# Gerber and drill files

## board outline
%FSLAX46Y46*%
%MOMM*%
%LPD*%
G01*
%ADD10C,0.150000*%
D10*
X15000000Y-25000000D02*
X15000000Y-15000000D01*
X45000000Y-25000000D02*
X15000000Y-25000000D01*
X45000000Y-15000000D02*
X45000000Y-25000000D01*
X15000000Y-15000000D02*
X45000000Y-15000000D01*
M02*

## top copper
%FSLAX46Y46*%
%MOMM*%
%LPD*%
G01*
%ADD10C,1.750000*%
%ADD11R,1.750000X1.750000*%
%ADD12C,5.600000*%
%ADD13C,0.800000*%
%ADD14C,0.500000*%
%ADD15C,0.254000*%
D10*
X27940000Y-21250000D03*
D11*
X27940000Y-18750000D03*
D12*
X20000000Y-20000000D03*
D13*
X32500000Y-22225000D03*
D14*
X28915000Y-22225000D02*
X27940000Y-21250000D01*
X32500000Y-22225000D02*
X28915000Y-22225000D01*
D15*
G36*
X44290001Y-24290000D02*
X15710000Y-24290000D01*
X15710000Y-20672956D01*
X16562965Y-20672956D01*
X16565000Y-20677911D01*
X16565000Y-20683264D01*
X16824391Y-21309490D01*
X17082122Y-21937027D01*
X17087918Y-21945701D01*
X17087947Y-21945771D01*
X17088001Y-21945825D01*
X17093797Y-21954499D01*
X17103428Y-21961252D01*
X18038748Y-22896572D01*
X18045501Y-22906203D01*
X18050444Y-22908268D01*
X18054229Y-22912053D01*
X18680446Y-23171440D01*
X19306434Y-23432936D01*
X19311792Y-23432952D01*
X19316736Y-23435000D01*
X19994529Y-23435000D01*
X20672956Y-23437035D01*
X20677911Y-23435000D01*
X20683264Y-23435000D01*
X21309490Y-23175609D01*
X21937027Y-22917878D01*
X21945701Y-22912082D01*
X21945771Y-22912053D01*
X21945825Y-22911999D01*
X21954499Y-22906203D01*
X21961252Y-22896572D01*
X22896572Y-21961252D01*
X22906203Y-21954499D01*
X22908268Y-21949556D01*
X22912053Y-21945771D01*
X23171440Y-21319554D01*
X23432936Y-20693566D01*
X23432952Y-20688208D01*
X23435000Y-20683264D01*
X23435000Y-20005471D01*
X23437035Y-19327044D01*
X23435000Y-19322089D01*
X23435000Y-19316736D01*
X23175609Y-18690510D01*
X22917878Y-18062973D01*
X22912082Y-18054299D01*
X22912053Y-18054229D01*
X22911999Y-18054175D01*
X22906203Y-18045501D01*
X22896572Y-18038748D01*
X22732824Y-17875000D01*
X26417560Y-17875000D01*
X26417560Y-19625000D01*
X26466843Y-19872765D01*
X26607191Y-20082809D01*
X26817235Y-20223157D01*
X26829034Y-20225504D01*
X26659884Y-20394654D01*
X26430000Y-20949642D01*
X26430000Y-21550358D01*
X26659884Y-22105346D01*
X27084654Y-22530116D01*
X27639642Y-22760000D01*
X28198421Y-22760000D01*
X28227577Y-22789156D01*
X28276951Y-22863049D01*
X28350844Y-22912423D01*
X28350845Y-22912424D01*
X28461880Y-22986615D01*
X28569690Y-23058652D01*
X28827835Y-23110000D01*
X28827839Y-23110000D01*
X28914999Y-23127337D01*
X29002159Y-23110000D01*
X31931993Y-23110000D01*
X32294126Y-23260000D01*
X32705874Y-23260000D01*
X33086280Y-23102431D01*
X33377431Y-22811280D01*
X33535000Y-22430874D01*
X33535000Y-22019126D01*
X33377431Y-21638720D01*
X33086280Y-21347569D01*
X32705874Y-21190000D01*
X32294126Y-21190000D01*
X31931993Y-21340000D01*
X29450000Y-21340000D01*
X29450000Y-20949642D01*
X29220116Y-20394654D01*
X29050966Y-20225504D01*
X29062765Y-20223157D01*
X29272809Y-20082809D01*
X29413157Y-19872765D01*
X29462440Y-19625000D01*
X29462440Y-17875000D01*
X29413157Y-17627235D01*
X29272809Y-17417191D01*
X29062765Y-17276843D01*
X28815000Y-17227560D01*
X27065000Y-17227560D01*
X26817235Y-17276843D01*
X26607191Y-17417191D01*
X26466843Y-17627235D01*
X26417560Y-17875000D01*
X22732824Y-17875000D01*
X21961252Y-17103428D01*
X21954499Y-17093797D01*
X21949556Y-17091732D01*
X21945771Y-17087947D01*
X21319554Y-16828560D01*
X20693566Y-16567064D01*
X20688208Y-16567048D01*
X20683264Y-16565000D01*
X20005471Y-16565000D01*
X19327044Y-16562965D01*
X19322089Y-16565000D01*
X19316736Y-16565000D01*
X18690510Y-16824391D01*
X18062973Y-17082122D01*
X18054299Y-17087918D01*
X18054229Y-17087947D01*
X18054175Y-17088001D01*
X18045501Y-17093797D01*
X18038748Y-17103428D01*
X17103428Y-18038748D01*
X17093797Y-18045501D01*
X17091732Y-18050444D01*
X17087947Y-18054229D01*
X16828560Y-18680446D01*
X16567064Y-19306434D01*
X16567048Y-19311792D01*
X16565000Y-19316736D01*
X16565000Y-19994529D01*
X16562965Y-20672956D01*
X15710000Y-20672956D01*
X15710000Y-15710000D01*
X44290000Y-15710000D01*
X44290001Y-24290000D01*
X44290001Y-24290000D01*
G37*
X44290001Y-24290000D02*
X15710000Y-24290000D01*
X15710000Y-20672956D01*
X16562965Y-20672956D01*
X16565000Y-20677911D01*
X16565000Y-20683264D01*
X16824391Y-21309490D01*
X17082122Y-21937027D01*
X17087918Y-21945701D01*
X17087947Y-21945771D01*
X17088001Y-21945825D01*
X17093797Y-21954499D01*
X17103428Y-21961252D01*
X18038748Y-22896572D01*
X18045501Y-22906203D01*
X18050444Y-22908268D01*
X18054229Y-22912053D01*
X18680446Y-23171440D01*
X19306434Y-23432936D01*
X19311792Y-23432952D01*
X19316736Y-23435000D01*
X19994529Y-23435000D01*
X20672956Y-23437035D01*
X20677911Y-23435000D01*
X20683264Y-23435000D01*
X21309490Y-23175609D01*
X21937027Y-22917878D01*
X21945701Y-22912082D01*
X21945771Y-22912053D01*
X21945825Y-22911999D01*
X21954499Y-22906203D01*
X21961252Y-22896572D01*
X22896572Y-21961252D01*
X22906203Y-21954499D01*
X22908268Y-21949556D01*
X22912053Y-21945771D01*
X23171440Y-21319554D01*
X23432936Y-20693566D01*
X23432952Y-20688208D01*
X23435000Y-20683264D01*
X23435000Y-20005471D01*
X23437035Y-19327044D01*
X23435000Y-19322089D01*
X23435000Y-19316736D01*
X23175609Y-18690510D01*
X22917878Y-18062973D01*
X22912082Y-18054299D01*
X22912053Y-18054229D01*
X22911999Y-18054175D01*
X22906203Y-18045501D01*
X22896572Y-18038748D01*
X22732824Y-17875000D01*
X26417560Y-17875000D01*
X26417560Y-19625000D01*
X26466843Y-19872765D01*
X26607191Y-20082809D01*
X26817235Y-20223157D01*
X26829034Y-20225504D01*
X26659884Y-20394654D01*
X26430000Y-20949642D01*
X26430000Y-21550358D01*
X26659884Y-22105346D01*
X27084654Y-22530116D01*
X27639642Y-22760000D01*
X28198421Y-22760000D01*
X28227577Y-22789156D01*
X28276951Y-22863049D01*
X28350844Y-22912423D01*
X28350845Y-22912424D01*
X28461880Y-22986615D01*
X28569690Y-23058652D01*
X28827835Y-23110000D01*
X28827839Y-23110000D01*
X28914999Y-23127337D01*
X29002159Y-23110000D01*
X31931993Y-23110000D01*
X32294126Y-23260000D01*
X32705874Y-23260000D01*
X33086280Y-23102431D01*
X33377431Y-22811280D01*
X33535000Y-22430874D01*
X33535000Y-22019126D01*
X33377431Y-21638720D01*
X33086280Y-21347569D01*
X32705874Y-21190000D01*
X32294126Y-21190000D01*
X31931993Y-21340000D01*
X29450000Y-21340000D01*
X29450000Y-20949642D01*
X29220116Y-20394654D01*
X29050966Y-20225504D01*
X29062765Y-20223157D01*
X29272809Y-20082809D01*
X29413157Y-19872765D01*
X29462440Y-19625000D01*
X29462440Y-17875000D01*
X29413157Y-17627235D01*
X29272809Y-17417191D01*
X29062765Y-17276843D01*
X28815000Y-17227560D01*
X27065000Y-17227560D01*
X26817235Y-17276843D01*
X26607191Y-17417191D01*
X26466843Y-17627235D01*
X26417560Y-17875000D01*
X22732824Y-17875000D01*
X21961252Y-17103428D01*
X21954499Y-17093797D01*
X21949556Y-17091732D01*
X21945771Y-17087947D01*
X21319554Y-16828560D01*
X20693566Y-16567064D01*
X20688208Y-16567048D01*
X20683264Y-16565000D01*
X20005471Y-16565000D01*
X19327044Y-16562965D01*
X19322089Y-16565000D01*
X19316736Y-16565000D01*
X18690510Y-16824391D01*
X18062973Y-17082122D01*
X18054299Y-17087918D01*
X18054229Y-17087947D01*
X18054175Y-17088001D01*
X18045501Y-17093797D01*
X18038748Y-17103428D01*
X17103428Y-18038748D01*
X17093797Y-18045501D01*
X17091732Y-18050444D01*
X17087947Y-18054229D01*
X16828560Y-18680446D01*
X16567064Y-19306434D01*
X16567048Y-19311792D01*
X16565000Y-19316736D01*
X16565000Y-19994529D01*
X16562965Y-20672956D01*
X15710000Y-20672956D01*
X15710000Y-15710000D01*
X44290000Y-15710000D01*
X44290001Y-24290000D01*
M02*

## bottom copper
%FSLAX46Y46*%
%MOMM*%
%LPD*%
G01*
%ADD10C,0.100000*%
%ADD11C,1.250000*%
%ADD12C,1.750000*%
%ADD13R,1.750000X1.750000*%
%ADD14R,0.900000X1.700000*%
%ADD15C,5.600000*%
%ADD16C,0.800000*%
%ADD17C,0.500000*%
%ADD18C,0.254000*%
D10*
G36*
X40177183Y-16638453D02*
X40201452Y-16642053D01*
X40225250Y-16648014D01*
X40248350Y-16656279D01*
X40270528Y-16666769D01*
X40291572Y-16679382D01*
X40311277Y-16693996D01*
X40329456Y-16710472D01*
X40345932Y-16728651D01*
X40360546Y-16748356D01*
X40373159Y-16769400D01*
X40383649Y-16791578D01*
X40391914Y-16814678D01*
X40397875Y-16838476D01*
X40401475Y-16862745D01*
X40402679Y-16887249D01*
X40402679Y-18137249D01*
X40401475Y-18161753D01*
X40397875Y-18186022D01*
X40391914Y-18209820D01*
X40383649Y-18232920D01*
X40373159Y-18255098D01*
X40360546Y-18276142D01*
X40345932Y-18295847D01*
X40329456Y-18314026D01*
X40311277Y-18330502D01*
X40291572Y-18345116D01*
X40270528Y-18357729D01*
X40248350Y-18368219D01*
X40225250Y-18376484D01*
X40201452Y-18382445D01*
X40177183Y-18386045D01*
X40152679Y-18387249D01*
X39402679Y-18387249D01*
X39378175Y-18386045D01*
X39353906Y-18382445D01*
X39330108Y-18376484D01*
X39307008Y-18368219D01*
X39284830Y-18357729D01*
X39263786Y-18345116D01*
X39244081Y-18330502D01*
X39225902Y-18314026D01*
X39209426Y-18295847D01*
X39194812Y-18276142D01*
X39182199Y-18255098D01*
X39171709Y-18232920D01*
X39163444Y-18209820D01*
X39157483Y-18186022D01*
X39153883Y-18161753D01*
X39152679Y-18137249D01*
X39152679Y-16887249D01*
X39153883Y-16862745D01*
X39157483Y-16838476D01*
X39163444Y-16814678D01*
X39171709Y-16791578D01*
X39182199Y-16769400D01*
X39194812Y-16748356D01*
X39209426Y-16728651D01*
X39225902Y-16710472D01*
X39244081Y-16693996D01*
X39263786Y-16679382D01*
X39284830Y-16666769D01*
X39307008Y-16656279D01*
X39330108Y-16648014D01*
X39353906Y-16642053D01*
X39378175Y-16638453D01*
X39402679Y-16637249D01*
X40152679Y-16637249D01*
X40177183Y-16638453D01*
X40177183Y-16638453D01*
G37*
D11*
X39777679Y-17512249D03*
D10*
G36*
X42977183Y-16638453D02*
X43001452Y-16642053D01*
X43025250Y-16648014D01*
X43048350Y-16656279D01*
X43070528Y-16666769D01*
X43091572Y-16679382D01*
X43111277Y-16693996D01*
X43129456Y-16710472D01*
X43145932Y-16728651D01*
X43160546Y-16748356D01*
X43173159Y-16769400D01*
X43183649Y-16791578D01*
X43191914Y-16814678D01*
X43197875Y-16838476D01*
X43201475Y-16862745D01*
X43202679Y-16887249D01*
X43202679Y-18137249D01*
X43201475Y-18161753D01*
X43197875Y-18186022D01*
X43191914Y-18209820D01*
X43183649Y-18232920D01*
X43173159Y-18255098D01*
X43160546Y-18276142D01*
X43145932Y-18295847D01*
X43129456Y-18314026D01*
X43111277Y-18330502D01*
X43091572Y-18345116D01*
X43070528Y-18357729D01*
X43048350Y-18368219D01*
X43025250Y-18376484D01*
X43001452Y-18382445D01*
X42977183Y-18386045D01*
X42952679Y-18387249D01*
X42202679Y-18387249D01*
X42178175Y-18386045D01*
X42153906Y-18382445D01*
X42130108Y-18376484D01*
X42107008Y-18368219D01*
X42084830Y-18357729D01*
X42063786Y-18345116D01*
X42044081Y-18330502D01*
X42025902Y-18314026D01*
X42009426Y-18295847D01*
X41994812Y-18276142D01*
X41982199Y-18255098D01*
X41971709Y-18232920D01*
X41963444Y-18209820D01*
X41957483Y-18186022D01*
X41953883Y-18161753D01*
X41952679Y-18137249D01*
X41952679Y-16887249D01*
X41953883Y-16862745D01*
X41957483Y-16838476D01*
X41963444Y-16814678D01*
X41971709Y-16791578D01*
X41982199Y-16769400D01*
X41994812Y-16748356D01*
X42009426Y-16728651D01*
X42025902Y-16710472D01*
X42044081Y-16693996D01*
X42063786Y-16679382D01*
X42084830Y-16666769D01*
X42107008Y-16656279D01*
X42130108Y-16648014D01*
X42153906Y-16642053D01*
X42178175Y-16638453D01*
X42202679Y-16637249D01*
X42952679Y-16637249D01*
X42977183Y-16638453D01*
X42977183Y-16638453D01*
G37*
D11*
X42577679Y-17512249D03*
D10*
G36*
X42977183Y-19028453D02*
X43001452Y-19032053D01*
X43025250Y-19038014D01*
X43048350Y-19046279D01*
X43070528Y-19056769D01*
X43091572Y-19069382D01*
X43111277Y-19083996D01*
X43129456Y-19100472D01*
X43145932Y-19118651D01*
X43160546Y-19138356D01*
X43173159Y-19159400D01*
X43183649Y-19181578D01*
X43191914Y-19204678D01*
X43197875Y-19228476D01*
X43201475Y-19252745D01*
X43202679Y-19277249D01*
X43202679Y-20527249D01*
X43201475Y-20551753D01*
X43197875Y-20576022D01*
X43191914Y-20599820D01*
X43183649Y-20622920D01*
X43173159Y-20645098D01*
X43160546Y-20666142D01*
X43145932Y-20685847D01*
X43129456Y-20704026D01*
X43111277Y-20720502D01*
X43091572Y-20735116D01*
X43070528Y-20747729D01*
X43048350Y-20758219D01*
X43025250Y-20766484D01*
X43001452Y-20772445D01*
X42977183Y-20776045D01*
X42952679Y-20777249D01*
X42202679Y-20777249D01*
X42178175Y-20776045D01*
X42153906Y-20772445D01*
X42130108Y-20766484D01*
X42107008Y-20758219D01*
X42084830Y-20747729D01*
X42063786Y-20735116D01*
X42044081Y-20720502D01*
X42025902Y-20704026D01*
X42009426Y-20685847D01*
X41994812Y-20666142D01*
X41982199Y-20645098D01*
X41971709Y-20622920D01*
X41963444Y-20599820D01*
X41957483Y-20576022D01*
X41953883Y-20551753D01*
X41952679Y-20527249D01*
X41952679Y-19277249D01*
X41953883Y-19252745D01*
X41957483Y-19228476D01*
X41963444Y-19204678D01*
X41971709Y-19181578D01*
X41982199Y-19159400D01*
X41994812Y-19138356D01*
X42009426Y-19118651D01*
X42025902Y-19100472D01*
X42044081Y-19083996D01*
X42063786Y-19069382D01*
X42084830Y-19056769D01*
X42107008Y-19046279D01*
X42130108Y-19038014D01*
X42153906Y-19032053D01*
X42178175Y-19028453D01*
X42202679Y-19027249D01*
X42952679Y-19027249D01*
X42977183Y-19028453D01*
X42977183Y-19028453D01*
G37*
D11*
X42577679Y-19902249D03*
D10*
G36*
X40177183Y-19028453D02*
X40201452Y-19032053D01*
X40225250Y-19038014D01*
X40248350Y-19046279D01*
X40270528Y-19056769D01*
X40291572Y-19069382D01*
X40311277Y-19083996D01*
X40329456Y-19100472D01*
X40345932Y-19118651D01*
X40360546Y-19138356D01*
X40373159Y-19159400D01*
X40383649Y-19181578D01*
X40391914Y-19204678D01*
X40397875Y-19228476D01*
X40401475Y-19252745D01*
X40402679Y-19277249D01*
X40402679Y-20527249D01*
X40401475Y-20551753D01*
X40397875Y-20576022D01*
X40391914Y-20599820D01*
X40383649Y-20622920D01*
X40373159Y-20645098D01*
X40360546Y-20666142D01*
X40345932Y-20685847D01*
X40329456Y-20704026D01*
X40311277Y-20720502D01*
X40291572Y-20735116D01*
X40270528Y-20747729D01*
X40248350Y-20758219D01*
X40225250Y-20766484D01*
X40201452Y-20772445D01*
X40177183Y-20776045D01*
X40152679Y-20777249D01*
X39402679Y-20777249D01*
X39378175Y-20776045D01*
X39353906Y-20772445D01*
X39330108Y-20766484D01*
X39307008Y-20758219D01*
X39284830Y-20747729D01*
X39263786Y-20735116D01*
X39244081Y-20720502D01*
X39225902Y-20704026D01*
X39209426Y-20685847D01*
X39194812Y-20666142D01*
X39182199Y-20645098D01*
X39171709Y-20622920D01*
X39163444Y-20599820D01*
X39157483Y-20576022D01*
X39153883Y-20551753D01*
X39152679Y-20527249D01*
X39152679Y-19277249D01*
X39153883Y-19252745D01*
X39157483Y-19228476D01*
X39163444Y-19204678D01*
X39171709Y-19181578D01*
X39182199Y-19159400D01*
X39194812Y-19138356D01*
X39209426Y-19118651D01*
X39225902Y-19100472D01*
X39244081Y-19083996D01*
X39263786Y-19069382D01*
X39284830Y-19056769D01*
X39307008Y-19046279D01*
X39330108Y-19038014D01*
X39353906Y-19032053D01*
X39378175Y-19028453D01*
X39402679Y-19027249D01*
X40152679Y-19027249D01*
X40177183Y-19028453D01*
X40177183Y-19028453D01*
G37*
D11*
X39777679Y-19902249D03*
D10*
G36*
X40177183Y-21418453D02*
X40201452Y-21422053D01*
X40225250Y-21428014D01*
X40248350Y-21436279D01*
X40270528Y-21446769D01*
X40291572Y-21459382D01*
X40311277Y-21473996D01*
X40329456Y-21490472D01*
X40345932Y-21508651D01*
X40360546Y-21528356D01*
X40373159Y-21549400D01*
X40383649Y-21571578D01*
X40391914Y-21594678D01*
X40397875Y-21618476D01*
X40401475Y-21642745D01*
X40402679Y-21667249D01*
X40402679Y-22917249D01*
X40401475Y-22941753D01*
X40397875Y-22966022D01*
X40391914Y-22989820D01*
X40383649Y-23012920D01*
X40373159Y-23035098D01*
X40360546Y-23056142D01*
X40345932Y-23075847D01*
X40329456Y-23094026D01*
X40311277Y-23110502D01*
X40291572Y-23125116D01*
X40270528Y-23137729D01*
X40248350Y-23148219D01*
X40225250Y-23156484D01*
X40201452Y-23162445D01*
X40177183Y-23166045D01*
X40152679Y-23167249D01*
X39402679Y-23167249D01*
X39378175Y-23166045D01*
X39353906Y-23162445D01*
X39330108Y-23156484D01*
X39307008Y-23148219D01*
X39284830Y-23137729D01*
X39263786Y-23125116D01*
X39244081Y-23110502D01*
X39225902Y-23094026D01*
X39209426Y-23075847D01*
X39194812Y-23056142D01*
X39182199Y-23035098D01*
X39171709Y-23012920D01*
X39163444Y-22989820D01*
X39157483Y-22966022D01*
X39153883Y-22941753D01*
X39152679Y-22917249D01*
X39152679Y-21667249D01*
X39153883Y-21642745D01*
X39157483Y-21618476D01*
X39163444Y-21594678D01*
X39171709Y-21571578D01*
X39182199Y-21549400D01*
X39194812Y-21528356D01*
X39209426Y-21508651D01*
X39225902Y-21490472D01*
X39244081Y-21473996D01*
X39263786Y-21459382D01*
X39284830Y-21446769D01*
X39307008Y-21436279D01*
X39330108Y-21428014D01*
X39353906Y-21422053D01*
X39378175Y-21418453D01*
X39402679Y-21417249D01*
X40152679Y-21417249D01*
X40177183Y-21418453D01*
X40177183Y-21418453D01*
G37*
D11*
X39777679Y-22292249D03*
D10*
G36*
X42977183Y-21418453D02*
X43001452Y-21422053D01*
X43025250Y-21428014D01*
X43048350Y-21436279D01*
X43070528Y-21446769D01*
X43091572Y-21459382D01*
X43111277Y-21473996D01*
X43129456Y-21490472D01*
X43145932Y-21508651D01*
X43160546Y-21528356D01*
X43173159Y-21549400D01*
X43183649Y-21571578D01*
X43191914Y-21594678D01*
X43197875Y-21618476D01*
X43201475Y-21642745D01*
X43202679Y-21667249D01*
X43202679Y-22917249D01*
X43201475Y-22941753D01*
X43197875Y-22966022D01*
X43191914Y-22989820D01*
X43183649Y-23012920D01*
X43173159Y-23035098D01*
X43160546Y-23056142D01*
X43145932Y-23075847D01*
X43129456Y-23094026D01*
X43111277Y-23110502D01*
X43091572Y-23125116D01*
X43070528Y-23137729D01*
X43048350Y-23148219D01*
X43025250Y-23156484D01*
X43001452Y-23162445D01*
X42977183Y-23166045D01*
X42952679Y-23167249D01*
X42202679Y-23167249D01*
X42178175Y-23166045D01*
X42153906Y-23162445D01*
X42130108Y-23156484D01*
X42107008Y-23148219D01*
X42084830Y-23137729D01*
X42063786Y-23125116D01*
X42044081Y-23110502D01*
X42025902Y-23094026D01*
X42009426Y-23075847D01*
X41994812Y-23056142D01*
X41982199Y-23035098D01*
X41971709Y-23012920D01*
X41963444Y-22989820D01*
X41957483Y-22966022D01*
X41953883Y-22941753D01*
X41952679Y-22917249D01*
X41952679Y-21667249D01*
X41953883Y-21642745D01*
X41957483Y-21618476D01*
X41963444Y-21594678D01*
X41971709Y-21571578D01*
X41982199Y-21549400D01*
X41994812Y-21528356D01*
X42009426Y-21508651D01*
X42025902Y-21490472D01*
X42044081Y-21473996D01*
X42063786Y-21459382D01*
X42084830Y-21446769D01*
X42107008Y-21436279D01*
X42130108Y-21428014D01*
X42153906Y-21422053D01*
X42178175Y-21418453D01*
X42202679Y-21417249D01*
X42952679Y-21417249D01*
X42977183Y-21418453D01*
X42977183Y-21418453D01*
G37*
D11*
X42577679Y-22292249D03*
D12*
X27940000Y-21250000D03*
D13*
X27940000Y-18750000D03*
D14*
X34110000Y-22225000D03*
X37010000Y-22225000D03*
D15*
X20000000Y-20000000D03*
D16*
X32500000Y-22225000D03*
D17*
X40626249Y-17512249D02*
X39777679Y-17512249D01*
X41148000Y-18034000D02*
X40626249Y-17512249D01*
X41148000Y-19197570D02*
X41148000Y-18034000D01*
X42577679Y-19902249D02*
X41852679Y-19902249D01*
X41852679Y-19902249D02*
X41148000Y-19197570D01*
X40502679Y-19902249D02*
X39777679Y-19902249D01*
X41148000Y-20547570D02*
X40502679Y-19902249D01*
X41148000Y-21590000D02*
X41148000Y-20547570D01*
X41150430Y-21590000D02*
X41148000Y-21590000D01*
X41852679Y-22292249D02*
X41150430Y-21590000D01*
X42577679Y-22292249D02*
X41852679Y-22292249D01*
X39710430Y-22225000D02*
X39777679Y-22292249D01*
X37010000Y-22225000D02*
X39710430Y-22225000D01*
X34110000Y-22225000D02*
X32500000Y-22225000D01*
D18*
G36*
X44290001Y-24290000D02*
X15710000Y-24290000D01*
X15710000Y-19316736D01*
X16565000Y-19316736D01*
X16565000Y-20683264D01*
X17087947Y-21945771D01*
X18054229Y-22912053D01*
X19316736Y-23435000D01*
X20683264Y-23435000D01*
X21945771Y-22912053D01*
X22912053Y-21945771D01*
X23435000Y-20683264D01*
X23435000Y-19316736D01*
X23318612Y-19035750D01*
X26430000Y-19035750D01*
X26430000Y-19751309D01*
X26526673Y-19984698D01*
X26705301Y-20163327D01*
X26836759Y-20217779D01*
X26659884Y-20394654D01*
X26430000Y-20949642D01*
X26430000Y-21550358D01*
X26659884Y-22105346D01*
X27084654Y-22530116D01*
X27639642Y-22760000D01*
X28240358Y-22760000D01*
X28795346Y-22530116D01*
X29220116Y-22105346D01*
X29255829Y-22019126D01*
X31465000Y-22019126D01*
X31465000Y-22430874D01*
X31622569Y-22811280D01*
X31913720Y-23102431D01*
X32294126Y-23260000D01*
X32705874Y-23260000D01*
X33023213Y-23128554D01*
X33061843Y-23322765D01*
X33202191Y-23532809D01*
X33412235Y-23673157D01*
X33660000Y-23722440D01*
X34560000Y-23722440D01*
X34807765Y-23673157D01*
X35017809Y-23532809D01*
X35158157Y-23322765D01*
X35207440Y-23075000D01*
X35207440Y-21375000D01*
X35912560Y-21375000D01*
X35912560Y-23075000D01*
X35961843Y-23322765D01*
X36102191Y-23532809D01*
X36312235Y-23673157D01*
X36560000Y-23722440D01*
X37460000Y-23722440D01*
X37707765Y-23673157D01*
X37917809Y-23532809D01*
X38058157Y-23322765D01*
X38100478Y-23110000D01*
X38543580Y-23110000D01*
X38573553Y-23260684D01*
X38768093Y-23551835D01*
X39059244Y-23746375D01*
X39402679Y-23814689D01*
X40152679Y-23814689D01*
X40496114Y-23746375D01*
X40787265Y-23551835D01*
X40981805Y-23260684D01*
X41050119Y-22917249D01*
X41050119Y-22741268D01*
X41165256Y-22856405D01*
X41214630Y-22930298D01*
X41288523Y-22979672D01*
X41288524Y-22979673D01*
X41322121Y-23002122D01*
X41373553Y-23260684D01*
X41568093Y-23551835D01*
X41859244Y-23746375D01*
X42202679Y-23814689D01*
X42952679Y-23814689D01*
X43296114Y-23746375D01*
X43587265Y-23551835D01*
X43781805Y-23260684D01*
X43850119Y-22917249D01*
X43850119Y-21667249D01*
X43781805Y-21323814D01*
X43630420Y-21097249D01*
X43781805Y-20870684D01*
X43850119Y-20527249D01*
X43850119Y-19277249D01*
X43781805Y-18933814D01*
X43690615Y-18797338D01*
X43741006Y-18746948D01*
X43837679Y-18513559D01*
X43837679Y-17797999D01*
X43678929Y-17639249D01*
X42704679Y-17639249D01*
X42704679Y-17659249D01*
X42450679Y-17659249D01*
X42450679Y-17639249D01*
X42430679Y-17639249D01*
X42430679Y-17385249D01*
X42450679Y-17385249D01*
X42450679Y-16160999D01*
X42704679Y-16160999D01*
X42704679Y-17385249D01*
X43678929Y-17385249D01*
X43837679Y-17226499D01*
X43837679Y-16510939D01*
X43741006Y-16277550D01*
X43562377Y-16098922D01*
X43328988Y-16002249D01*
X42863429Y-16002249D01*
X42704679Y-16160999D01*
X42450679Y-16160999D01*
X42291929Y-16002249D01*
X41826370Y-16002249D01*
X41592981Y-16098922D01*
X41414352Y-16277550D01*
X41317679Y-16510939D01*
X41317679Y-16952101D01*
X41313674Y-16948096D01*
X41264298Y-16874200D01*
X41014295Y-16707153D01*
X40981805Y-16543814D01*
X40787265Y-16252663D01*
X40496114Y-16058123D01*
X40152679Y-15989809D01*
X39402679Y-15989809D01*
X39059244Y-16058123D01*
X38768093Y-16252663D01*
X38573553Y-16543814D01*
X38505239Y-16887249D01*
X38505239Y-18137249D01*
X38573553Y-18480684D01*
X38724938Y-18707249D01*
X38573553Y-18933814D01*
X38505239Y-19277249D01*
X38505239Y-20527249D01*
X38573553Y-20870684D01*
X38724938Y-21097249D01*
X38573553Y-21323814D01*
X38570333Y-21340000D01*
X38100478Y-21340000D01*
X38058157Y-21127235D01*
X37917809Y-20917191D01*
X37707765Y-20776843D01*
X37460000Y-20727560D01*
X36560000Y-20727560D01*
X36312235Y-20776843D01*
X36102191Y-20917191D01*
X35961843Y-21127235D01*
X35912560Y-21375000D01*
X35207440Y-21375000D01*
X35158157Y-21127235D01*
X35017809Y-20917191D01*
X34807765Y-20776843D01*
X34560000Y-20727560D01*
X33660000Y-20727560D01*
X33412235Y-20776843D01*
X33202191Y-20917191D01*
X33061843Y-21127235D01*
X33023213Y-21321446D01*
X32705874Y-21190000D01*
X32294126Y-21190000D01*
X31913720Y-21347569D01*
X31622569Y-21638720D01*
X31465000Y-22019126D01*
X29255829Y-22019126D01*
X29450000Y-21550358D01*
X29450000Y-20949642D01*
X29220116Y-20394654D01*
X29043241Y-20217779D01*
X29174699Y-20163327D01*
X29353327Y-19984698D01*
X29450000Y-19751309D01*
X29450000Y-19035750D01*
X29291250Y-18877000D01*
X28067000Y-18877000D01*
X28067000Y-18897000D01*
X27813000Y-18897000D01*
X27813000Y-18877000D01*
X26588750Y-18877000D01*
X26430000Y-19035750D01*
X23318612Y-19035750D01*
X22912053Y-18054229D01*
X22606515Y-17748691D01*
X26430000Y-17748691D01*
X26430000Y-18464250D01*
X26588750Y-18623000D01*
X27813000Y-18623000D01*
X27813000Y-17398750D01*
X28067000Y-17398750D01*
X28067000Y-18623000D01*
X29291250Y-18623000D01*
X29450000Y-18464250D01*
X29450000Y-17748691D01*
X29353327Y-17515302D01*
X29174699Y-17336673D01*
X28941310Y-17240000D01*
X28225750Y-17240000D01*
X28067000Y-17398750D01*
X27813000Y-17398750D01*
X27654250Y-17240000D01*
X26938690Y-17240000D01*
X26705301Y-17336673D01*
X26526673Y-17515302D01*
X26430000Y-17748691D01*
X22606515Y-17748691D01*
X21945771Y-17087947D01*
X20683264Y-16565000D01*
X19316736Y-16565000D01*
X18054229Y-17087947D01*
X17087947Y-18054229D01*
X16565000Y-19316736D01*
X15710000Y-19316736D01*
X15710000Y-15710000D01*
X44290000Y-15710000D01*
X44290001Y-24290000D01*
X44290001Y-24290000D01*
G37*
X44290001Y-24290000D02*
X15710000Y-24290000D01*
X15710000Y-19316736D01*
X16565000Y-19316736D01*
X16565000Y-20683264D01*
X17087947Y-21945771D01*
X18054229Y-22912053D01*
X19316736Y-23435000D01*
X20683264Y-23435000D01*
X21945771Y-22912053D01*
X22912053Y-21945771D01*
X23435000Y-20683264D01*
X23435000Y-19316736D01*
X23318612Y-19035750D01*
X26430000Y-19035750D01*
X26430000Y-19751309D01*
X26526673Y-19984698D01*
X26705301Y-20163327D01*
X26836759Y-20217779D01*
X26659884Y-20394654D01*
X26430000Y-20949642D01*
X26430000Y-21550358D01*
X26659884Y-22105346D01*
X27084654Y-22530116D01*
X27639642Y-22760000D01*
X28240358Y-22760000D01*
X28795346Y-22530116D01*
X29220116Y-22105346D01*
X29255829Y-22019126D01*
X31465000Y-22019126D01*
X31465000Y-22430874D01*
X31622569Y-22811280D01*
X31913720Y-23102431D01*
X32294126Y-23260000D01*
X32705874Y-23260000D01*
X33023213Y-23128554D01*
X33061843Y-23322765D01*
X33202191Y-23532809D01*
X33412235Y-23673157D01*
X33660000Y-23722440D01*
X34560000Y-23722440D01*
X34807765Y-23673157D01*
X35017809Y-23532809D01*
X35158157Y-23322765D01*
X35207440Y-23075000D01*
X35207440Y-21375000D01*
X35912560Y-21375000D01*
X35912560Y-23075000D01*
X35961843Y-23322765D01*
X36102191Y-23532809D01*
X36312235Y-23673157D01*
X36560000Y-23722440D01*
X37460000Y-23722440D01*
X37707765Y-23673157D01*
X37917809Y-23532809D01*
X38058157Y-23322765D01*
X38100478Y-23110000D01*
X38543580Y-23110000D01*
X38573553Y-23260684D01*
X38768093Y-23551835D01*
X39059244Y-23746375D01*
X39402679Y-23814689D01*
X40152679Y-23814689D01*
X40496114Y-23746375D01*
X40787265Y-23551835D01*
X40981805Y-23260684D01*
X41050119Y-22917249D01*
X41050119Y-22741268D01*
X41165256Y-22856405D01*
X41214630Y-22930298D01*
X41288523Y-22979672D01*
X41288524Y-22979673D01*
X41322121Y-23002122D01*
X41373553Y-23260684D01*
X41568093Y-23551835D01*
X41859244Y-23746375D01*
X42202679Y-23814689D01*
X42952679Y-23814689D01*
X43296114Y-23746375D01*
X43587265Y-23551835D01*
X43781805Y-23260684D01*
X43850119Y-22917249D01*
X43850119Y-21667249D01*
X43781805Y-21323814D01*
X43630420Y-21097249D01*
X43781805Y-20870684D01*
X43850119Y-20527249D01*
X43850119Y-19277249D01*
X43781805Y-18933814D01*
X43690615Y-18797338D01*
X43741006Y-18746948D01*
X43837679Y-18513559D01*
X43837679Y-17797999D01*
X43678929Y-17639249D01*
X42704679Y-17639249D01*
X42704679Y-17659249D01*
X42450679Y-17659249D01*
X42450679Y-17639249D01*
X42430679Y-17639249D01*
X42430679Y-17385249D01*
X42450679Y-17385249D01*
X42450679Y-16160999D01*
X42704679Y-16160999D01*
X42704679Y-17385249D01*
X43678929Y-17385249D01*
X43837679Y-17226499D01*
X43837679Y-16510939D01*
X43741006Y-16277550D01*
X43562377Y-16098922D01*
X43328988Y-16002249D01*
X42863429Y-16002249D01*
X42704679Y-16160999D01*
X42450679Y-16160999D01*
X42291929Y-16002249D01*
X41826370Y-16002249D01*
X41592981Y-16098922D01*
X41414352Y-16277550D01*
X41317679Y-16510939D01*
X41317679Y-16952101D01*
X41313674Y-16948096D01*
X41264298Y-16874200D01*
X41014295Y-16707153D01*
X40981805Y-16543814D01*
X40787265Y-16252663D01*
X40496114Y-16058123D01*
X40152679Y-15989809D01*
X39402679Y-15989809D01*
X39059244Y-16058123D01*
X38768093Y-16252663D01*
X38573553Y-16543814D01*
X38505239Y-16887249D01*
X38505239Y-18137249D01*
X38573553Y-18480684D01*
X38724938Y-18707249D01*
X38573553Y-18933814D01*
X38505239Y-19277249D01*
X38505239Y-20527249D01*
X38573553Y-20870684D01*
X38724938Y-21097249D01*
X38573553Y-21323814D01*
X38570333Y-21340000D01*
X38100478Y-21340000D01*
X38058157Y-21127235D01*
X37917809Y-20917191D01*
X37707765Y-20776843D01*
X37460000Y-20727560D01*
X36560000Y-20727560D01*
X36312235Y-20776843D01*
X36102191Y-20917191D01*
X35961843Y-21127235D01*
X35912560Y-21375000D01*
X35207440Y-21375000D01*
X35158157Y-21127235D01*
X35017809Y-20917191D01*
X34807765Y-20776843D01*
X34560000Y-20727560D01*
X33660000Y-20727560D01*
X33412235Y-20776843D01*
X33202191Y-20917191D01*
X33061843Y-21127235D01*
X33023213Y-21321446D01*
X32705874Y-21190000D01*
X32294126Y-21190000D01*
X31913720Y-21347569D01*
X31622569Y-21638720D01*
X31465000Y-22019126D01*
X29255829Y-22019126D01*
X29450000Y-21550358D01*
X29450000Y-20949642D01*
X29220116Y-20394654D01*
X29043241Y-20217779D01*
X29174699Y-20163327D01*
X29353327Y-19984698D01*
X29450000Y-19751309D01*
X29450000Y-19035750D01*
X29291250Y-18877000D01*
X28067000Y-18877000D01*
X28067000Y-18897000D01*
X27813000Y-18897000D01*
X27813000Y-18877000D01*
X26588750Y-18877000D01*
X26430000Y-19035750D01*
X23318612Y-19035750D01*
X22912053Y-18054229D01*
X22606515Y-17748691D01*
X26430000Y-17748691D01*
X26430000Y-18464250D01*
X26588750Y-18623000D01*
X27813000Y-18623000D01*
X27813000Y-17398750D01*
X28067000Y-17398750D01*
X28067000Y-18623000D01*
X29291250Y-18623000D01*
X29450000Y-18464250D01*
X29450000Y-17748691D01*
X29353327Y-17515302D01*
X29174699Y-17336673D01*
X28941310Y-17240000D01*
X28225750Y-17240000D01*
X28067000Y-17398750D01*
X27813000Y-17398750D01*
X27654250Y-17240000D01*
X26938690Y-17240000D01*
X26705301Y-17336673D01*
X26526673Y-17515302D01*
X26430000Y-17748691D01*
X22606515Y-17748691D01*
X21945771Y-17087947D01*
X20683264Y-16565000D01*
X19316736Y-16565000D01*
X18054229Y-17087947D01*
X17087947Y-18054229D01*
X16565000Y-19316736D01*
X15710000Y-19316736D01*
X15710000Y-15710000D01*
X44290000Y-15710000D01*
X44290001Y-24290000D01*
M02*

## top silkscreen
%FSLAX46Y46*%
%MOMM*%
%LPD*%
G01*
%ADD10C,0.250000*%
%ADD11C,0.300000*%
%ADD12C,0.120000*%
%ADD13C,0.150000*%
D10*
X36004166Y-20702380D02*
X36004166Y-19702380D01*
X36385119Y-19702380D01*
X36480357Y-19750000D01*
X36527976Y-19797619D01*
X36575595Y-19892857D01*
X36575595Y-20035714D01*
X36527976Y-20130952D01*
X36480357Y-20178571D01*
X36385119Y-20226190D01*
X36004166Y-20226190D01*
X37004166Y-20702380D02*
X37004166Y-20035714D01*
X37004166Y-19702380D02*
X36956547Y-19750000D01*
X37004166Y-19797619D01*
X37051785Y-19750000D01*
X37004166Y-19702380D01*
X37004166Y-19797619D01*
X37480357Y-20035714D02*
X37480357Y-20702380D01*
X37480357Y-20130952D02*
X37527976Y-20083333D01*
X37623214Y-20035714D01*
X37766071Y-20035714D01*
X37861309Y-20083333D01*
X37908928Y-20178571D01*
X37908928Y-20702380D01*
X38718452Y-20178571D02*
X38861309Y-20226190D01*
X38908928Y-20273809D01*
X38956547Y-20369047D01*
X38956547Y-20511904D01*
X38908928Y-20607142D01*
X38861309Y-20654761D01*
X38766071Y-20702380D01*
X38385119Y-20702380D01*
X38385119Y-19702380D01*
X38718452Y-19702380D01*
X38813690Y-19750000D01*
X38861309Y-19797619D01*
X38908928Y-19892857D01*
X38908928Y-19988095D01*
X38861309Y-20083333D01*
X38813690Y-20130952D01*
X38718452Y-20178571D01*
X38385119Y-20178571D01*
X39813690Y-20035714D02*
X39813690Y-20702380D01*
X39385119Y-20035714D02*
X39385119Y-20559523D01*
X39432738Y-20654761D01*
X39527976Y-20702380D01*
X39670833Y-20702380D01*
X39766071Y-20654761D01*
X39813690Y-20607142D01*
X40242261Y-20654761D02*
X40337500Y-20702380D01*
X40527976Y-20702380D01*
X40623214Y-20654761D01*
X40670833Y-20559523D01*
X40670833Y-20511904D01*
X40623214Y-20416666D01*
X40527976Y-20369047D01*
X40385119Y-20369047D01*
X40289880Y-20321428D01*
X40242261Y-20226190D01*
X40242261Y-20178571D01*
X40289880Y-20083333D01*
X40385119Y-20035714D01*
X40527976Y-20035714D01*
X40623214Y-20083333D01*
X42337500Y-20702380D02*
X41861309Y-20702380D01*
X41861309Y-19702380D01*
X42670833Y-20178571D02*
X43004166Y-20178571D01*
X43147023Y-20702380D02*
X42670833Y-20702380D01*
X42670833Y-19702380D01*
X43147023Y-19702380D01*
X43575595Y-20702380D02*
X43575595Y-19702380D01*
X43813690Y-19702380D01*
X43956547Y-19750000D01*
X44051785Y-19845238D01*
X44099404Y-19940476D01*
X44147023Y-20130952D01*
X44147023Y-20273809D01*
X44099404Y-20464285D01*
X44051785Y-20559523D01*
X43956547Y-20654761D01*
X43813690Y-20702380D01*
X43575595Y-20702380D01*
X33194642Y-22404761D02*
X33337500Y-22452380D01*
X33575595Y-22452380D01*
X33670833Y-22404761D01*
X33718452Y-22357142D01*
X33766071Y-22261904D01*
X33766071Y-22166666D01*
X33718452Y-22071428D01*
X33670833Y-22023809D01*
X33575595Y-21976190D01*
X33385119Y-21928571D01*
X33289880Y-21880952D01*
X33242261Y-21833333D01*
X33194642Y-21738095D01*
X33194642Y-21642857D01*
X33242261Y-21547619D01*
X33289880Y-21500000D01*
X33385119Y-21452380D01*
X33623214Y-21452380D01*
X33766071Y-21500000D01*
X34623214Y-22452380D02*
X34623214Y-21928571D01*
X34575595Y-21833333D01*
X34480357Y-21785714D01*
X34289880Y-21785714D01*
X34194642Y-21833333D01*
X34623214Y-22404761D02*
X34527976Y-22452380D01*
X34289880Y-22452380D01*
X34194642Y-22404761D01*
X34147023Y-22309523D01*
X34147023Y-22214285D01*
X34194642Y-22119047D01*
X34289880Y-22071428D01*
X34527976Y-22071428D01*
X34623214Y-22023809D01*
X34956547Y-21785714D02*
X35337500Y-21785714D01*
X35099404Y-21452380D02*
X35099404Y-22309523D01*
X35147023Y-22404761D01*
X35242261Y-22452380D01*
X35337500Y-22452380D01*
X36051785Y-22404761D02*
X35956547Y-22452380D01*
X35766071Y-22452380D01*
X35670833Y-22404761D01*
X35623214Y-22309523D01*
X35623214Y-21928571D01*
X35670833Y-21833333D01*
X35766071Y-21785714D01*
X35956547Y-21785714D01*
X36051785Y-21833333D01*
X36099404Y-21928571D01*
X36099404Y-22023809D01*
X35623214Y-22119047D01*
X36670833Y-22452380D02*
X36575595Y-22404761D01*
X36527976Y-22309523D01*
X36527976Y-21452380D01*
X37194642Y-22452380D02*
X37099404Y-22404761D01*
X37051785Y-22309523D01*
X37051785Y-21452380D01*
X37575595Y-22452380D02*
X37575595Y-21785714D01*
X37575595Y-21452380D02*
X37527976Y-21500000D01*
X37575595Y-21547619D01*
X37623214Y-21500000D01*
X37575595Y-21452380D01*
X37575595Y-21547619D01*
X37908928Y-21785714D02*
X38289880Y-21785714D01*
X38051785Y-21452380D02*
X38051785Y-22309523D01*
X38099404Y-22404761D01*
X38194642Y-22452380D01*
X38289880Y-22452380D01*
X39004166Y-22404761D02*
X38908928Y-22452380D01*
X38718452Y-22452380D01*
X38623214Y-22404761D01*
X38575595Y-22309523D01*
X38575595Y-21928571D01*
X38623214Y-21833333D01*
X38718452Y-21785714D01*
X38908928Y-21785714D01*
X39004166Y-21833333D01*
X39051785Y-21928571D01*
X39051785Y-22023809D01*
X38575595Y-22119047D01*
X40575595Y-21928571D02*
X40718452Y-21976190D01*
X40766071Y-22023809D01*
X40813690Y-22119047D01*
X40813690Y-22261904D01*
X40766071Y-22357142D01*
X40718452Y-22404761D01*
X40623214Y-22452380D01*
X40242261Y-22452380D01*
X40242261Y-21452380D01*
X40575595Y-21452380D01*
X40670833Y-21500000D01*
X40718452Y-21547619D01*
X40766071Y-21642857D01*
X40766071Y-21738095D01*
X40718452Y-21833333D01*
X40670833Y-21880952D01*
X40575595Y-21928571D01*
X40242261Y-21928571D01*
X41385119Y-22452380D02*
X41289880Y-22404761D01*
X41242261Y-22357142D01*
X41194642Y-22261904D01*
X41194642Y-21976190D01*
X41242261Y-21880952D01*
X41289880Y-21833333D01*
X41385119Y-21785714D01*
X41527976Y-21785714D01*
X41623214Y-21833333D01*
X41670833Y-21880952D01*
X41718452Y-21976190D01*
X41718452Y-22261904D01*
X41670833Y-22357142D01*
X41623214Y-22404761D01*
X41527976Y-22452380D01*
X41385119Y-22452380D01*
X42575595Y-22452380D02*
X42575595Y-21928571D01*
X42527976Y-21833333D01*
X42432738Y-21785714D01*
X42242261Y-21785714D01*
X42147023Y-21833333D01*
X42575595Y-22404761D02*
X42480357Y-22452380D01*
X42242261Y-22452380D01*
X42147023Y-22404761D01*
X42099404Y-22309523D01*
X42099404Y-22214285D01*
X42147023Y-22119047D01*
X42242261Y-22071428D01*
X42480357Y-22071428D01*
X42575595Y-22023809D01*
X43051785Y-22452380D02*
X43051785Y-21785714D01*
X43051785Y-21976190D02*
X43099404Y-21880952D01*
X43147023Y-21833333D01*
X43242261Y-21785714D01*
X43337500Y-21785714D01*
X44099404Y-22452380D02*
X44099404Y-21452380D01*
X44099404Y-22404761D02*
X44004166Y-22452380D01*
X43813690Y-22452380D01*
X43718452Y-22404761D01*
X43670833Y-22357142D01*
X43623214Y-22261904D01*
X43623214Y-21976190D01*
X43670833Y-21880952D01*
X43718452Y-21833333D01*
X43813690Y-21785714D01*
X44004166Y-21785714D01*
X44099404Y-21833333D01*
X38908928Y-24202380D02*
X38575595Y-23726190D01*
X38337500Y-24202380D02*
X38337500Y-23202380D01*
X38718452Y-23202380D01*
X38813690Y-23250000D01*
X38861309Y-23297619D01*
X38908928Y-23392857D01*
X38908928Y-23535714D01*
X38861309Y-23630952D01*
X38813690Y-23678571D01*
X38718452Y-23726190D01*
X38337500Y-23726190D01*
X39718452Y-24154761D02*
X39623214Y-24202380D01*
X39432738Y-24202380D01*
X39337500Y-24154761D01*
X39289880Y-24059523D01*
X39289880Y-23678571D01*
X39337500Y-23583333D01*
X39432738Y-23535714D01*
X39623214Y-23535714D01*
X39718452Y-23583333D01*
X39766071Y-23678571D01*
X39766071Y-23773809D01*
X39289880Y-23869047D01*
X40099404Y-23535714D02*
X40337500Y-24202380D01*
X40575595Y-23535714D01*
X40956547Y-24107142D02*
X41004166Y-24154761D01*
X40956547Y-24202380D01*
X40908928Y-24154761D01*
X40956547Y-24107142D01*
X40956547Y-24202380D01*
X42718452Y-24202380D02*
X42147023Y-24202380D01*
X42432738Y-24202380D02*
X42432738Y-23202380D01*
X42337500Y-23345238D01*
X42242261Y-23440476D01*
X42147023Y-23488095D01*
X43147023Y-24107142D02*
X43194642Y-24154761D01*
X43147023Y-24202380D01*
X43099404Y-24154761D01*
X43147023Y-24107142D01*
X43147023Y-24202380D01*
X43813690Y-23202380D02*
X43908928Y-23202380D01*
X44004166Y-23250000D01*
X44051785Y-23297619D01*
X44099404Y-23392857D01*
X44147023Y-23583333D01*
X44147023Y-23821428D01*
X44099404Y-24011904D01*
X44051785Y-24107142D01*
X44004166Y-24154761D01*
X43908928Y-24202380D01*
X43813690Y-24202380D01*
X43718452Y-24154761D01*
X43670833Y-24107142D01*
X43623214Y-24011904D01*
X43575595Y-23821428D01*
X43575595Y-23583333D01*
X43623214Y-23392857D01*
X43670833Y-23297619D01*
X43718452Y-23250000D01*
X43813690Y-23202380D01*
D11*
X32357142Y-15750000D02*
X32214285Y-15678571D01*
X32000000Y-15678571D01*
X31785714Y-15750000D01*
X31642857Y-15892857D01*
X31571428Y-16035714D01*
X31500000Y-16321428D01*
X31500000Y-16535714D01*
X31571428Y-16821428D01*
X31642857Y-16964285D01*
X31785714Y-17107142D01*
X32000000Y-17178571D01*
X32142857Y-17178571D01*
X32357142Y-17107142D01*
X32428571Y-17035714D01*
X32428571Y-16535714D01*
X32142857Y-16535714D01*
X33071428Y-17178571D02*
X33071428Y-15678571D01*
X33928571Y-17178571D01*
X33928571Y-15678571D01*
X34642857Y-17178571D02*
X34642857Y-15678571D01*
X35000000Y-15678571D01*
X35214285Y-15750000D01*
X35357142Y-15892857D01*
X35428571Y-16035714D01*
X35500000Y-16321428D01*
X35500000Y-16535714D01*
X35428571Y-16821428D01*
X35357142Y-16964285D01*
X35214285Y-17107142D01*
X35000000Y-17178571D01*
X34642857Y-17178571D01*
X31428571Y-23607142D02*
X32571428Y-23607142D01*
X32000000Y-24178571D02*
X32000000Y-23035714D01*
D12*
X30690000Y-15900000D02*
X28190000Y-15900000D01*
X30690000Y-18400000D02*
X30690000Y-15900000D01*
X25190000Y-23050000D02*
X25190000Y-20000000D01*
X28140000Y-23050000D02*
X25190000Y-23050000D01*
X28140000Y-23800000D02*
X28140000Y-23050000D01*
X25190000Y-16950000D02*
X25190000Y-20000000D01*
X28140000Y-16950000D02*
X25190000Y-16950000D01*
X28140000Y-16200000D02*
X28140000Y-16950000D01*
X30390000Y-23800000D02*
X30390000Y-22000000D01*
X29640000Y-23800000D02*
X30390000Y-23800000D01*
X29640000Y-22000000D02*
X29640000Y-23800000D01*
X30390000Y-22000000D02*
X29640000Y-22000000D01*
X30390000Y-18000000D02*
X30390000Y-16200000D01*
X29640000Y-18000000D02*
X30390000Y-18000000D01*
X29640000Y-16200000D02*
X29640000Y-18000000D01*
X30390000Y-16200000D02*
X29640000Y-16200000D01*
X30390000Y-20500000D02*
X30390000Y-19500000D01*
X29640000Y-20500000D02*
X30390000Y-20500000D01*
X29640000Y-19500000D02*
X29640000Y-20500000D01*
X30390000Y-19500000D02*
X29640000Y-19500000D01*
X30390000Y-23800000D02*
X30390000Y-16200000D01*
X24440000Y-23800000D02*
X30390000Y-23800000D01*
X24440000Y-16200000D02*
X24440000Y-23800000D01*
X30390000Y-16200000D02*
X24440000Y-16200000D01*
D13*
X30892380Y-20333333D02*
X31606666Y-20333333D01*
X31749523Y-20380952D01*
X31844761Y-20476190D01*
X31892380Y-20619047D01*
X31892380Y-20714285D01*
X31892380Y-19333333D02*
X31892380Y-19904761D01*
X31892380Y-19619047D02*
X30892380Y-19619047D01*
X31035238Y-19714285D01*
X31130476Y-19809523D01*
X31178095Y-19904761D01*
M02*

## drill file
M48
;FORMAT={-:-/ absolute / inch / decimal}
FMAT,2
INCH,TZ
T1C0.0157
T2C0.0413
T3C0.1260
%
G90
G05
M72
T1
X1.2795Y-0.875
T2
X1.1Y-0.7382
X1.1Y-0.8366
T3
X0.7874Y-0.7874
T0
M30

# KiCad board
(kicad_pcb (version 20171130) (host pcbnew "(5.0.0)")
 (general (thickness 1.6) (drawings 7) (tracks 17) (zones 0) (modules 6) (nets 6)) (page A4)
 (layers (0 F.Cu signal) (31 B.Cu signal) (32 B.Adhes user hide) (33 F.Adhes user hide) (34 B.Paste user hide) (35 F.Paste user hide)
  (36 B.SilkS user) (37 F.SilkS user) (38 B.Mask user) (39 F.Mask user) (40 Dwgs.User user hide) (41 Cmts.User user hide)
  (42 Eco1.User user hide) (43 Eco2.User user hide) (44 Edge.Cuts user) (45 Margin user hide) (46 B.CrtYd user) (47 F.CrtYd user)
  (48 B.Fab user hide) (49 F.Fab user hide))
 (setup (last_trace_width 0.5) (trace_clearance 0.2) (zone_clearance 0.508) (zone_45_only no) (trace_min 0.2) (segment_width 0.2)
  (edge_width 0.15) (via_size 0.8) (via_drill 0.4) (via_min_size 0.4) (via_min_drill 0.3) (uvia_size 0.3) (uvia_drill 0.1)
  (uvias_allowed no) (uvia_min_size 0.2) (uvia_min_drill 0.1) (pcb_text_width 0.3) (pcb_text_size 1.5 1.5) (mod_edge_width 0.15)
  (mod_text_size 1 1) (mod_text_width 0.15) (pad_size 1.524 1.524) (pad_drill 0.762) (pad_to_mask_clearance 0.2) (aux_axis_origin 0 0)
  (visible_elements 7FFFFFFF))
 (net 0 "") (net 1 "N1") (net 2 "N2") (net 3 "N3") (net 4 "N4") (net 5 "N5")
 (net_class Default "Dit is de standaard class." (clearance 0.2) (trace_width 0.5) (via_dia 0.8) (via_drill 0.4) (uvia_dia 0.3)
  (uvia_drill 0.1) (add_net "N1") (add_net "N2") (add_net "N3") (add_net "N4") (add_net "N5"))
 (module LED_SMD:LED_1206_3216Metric (layer B.Cu) (at 41.177679 17.512249)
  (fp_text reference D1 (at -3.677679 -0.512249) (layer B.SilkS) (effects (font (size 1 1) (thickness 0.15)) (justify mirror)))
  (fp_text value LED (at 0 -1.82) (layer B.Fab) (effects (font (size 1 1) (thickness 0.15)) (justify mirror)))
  (pad 1 smd roundrect (at -1.4 0) (size 1.25 1.75) (layers B.Cu B.Paste B.Mask) (roundrect_rratio 0.2) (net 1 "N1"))
  (pad 2 smd roundrect (at 1.4 0) (size 1.25 1.75) (layers B.Cu B.Paste B.Mask) (roundrect_rratio 0.2) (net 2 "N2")))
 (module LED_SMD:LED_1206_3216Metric (layer B.Cu) (at 41.177679 19.902249)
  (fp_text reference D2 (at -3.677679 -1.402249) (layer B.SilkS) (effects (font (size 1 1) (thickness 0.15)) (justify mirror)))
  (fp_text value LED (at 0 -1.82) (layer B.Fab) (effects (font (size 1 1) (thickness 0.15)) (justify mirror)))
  (pad 2 smd roundrect (at 1.4 0) (size 1.25 1.75) (layers B.Cu B.Paste B.Mask) (roundrect_rratio 0.2) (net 1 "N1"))
  (pad 1 smd roundrect (at -1.4 0) (size 1.25 1.75) (layers B.Cu B.Paste B.Mask) (roundrect_rratio 0.2) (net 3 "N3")))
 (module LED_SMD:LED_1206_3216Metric (layer B.Cu) (at 41.177679 22.292249)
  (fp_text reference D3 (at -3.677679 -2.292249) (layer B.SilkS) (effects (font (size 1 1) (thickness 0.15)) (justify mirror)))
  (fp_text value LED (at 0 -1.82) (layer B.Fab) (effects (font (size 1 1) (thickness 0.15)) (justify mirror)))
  (pad 1 smd roundrect (at -1.4 0) (size 1.25 1.75) (layers B.Cu B.Paste B.Mask) (roundrect_rratio 0.2) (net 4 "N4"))
  (pad 2 smd roundrect (at 1.4 0) (size 1.25 1.75) (layers B.Cu B.Paste B.Mask) (roundrect_rratio 0.2) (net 3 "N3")))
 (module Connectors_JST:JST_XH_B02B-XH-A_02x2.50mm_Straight (layer F.Cu) (at 27.94 18.75 270)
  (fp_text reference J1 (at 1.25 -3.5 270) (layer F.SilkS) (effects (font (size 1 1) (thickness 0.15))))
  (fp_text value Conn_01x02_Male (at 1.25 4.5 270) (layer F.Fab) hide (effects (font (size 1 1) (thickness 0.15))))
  (fp_line (start -2.85 -2.75) (end -2.85 -0.25) (layer F.SilkS) (width 0.12))
  (fp_line (start -0.35 -2.75) (end -2.85 -2.75) (layer F.SilkS) (width 0.12))
  (fp_line (start 4.3 2.75) (end 1.25 2.75) (layer F.SilkS) (width 0.12))
  (fp_line (start 4.3 -0.2) (end 4.3 2.75) (layer F.SilkS) (width 0.12))
  (fp_line (start 5.05 -0.2) (end 4.3 -0.2) (layer F.SilkS) (width 0.12))
  (fp_line (start -1.8 2.75) (end 1.25 2.75) (layer F.SilkS) (width 0.12))
  (fp_line (start -1.8 -0.2) (end -1.8 2.75) (layer F.SilkS) (width 0.12))
  (fp_line (start -2.55 -0.2) (end -1.8 -0.2) (layer F.SilkS) (width 0.12))
  (fp_line (start 5.05 -2.45) (end 3.25 -2.45) (layer F.SilkS) (width 0.12))
  (fp_line (start 5.05 -1.7) (end 5.05 -2.45) (layer F.SilkS) (width 0.12))
  (fp_line (start 3.25 -1.7) (end 5.05 -1.7) (layer F.SilkS) (width 0.12))
  (fp_line (start 3.25 -2.45) (end 3.25 -1.7) (layer F.SilkS) (width 0.12))
  (fp_line (start -0.75 -2.45) (end -2.55 -2.45) (layer F.SilkS) (width 0.12))
  (fp_line (start -0.75 -1.7) (end -0.75 -2.45) (layer F.SilkS) (width 0.12))
  (fp_line (start -2.55 -1.7) (end -0.75 -1.7) (layer F.SilkS) (width 0.12))
  (fp_line (start -2.55 -2.45) (end -2.55 -1.7) (layer F.SilkS) (width 0.12))
  (fp_line (start 1.75 -2.45) (end 0.75 -2.45) (layer F.SilkS) (width 0.12))
  (fp_line (start 1.75 -1.7) (end 1.75 -2.45) (layer F.SilkS) (width 0.12))
  (fp_line (start 0.75 -1.7) (end 1.75 -1.7) (layer F.SilkS) (width 0.12))
  (fp_line (start 0.75 -2.45) (end 0.75 -1.7) (layer F.SilkS) (width 0.12))
  (fp_line (start 5.05 -2.45) (end -2.55 -2.45) (layer F.SilkS) (width 0.12))
  (fp_line (start 5.05 3.5) (end 5.05 -2.45) (layer F.SilkS) (width 0.12))
  (fp_line (start -2.55 3.5) (end 5.05 3.5) (layer F.SilkS) (width 0.12))
  (fp_line (start -2.55 -2.45) (end -2.55 3.5) (layer F.SilkS) (width 0.12))
  (pad 2 thru_hole circle (at 2.5 0 270) (size 1.75 1.75) (drill 1.05) (layers *.Cu *.Mask) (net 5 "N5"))
  (pad 1 thru_hole rect (at 0 0 270) (size 1.75 1.75) (drill 1.05) (layers *.Cu *.Mask) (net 2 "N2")))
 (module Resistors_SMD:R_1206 (layer B.Cu) (at 35.56 22.225 180)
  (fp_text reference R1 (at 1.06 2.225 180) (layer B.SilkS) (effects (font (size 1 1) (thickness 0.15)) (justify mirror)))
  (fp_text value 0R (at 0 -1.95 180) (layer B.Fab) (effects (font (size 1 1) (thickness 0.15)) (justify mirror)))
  (pad 2 smd rect (at 1.45 0 180) (size 0.9 1.7) (layers B.Cu B.Paste B.Mask) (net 5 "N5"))
  (pad 1 smd rect (at -1.45 0 180) (size 0.9 1.7) (layers B.Cu B.Paste B.Mask) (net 4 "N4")))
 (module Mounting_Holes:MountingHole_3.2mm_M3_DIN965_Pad (layer F.Cu) (at 20 20)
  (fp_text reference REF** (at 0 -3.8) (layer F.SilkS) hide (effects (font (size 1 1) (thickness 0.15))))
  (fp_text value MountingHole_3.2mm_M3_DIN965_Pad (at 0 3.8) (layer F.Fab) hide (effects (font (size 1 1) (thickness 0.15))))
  (pad 1 thru_hole circle (at 0 0) (size 5.6 5.6) (drill 3.2) (layers *.Cu *.Mask)))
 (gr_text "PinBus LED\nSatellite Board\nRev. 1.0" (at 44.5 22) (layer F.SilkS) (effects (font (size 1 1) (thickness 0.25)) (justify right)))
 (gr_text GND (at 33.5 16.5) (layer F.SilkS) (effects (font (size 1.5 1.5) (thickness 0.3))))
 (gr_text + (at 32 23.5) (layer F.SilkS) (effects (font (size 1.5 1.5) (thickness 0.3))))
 (gr_line (start 15 25) (end 15 15) (layer Edge.Cuts) (width 0.15))
 (gr_line (start 45 25) (end 15 25) (layer Edge.Cuts) (width 0.15))
 (gr_line (start 45 15) (end 45 25) (layer Edge.Cuts) (width 0.15))
 (gr_line (start 15 15) (end 45 15) (layer Edge.Cuts) (width 0.15))
 (segment (start 40.626249 17.512249) (end 39.777679 17.512249) (width 0.5) (layer B.Cu) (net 1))
 (segment (start 41.148 18.034) (end 40.626249 17.512249) (width 0.5) (layer B.Cu) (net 1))
 (segment (start 41.148 19.19757) (end 41.148 18.034) (width 0.5) (layer B.Cu) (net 1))
 (segment (start 42.577679 19.902249) (end 41.852679 19.902249) (width 0.5) (layer B.Cu) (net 1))
 (segment (start 41.852679 19.902249) (end 41.148 19.19757) (width 0.5) (layer B.Cu) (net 1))
 (segment (start 40.502679 19.902249) (end 39.777679 19.902249) (width 0.5) (layer B.Cu) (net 3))
 (segment (start 41.148 20.54757) (end 40.502679 19.902249) (width 0.5) (layer B.Cu) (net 3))
 (segment (start 41.148 21.59) (end 41.148 20.54757) (width 0.5) (layer B.Cu) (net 3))
 (segment (start 41.15043 21.59) (end 41.148 21.59) (width 0.5) (layer B.Cu) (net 3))
 (segment (start 41.852679 22.292249) (end 41.15043 21.59) (width 0.5) (layer B.Cu) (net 3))
 (segment (start 42.577679 22.292249) (end 41.852679 22.292249) (width 0.5) (layer B.Cu) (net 3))
 (segment (start 39.71043 22.225) (end 39.777679 22.292249) (width 0.5) (layer B.Cu) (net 4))
 (segment (start 37.01 22.225) (end 39.71043 22.225) (width 0.5) (layer B.Cu) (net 4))
 (segment (start 34.11 22.225) (end 32.5 22.225) (width 0.5) (layer B.Cu) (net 5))
 (via (at 32.5 22.225) (size 0.8) (drill 0.4) (layers F.Cu B.Cu) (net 5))
 (segment (start 28.915 22.225) (end 27.94 21.25) (width 0.5) (layer F.Cu) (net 5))
 (segment (start 32.5 22.225) (end 28.915 22.225) (width 0.5) (layer F.Cu) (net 5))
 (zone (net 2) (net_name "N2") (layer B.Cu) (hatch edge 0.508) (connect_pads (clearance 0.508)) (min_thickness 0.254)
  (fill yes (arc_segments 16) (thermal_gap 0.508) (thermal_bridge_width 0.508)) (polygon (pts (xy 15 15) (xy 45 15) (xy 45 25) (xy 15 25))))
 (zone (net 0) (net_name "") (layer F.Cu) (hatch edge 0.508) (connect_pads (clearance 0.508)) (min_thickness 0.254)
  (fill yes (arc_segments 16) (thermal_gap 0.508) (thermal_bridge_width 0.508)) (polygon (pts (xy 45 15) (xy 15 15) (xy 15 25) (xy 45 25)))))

